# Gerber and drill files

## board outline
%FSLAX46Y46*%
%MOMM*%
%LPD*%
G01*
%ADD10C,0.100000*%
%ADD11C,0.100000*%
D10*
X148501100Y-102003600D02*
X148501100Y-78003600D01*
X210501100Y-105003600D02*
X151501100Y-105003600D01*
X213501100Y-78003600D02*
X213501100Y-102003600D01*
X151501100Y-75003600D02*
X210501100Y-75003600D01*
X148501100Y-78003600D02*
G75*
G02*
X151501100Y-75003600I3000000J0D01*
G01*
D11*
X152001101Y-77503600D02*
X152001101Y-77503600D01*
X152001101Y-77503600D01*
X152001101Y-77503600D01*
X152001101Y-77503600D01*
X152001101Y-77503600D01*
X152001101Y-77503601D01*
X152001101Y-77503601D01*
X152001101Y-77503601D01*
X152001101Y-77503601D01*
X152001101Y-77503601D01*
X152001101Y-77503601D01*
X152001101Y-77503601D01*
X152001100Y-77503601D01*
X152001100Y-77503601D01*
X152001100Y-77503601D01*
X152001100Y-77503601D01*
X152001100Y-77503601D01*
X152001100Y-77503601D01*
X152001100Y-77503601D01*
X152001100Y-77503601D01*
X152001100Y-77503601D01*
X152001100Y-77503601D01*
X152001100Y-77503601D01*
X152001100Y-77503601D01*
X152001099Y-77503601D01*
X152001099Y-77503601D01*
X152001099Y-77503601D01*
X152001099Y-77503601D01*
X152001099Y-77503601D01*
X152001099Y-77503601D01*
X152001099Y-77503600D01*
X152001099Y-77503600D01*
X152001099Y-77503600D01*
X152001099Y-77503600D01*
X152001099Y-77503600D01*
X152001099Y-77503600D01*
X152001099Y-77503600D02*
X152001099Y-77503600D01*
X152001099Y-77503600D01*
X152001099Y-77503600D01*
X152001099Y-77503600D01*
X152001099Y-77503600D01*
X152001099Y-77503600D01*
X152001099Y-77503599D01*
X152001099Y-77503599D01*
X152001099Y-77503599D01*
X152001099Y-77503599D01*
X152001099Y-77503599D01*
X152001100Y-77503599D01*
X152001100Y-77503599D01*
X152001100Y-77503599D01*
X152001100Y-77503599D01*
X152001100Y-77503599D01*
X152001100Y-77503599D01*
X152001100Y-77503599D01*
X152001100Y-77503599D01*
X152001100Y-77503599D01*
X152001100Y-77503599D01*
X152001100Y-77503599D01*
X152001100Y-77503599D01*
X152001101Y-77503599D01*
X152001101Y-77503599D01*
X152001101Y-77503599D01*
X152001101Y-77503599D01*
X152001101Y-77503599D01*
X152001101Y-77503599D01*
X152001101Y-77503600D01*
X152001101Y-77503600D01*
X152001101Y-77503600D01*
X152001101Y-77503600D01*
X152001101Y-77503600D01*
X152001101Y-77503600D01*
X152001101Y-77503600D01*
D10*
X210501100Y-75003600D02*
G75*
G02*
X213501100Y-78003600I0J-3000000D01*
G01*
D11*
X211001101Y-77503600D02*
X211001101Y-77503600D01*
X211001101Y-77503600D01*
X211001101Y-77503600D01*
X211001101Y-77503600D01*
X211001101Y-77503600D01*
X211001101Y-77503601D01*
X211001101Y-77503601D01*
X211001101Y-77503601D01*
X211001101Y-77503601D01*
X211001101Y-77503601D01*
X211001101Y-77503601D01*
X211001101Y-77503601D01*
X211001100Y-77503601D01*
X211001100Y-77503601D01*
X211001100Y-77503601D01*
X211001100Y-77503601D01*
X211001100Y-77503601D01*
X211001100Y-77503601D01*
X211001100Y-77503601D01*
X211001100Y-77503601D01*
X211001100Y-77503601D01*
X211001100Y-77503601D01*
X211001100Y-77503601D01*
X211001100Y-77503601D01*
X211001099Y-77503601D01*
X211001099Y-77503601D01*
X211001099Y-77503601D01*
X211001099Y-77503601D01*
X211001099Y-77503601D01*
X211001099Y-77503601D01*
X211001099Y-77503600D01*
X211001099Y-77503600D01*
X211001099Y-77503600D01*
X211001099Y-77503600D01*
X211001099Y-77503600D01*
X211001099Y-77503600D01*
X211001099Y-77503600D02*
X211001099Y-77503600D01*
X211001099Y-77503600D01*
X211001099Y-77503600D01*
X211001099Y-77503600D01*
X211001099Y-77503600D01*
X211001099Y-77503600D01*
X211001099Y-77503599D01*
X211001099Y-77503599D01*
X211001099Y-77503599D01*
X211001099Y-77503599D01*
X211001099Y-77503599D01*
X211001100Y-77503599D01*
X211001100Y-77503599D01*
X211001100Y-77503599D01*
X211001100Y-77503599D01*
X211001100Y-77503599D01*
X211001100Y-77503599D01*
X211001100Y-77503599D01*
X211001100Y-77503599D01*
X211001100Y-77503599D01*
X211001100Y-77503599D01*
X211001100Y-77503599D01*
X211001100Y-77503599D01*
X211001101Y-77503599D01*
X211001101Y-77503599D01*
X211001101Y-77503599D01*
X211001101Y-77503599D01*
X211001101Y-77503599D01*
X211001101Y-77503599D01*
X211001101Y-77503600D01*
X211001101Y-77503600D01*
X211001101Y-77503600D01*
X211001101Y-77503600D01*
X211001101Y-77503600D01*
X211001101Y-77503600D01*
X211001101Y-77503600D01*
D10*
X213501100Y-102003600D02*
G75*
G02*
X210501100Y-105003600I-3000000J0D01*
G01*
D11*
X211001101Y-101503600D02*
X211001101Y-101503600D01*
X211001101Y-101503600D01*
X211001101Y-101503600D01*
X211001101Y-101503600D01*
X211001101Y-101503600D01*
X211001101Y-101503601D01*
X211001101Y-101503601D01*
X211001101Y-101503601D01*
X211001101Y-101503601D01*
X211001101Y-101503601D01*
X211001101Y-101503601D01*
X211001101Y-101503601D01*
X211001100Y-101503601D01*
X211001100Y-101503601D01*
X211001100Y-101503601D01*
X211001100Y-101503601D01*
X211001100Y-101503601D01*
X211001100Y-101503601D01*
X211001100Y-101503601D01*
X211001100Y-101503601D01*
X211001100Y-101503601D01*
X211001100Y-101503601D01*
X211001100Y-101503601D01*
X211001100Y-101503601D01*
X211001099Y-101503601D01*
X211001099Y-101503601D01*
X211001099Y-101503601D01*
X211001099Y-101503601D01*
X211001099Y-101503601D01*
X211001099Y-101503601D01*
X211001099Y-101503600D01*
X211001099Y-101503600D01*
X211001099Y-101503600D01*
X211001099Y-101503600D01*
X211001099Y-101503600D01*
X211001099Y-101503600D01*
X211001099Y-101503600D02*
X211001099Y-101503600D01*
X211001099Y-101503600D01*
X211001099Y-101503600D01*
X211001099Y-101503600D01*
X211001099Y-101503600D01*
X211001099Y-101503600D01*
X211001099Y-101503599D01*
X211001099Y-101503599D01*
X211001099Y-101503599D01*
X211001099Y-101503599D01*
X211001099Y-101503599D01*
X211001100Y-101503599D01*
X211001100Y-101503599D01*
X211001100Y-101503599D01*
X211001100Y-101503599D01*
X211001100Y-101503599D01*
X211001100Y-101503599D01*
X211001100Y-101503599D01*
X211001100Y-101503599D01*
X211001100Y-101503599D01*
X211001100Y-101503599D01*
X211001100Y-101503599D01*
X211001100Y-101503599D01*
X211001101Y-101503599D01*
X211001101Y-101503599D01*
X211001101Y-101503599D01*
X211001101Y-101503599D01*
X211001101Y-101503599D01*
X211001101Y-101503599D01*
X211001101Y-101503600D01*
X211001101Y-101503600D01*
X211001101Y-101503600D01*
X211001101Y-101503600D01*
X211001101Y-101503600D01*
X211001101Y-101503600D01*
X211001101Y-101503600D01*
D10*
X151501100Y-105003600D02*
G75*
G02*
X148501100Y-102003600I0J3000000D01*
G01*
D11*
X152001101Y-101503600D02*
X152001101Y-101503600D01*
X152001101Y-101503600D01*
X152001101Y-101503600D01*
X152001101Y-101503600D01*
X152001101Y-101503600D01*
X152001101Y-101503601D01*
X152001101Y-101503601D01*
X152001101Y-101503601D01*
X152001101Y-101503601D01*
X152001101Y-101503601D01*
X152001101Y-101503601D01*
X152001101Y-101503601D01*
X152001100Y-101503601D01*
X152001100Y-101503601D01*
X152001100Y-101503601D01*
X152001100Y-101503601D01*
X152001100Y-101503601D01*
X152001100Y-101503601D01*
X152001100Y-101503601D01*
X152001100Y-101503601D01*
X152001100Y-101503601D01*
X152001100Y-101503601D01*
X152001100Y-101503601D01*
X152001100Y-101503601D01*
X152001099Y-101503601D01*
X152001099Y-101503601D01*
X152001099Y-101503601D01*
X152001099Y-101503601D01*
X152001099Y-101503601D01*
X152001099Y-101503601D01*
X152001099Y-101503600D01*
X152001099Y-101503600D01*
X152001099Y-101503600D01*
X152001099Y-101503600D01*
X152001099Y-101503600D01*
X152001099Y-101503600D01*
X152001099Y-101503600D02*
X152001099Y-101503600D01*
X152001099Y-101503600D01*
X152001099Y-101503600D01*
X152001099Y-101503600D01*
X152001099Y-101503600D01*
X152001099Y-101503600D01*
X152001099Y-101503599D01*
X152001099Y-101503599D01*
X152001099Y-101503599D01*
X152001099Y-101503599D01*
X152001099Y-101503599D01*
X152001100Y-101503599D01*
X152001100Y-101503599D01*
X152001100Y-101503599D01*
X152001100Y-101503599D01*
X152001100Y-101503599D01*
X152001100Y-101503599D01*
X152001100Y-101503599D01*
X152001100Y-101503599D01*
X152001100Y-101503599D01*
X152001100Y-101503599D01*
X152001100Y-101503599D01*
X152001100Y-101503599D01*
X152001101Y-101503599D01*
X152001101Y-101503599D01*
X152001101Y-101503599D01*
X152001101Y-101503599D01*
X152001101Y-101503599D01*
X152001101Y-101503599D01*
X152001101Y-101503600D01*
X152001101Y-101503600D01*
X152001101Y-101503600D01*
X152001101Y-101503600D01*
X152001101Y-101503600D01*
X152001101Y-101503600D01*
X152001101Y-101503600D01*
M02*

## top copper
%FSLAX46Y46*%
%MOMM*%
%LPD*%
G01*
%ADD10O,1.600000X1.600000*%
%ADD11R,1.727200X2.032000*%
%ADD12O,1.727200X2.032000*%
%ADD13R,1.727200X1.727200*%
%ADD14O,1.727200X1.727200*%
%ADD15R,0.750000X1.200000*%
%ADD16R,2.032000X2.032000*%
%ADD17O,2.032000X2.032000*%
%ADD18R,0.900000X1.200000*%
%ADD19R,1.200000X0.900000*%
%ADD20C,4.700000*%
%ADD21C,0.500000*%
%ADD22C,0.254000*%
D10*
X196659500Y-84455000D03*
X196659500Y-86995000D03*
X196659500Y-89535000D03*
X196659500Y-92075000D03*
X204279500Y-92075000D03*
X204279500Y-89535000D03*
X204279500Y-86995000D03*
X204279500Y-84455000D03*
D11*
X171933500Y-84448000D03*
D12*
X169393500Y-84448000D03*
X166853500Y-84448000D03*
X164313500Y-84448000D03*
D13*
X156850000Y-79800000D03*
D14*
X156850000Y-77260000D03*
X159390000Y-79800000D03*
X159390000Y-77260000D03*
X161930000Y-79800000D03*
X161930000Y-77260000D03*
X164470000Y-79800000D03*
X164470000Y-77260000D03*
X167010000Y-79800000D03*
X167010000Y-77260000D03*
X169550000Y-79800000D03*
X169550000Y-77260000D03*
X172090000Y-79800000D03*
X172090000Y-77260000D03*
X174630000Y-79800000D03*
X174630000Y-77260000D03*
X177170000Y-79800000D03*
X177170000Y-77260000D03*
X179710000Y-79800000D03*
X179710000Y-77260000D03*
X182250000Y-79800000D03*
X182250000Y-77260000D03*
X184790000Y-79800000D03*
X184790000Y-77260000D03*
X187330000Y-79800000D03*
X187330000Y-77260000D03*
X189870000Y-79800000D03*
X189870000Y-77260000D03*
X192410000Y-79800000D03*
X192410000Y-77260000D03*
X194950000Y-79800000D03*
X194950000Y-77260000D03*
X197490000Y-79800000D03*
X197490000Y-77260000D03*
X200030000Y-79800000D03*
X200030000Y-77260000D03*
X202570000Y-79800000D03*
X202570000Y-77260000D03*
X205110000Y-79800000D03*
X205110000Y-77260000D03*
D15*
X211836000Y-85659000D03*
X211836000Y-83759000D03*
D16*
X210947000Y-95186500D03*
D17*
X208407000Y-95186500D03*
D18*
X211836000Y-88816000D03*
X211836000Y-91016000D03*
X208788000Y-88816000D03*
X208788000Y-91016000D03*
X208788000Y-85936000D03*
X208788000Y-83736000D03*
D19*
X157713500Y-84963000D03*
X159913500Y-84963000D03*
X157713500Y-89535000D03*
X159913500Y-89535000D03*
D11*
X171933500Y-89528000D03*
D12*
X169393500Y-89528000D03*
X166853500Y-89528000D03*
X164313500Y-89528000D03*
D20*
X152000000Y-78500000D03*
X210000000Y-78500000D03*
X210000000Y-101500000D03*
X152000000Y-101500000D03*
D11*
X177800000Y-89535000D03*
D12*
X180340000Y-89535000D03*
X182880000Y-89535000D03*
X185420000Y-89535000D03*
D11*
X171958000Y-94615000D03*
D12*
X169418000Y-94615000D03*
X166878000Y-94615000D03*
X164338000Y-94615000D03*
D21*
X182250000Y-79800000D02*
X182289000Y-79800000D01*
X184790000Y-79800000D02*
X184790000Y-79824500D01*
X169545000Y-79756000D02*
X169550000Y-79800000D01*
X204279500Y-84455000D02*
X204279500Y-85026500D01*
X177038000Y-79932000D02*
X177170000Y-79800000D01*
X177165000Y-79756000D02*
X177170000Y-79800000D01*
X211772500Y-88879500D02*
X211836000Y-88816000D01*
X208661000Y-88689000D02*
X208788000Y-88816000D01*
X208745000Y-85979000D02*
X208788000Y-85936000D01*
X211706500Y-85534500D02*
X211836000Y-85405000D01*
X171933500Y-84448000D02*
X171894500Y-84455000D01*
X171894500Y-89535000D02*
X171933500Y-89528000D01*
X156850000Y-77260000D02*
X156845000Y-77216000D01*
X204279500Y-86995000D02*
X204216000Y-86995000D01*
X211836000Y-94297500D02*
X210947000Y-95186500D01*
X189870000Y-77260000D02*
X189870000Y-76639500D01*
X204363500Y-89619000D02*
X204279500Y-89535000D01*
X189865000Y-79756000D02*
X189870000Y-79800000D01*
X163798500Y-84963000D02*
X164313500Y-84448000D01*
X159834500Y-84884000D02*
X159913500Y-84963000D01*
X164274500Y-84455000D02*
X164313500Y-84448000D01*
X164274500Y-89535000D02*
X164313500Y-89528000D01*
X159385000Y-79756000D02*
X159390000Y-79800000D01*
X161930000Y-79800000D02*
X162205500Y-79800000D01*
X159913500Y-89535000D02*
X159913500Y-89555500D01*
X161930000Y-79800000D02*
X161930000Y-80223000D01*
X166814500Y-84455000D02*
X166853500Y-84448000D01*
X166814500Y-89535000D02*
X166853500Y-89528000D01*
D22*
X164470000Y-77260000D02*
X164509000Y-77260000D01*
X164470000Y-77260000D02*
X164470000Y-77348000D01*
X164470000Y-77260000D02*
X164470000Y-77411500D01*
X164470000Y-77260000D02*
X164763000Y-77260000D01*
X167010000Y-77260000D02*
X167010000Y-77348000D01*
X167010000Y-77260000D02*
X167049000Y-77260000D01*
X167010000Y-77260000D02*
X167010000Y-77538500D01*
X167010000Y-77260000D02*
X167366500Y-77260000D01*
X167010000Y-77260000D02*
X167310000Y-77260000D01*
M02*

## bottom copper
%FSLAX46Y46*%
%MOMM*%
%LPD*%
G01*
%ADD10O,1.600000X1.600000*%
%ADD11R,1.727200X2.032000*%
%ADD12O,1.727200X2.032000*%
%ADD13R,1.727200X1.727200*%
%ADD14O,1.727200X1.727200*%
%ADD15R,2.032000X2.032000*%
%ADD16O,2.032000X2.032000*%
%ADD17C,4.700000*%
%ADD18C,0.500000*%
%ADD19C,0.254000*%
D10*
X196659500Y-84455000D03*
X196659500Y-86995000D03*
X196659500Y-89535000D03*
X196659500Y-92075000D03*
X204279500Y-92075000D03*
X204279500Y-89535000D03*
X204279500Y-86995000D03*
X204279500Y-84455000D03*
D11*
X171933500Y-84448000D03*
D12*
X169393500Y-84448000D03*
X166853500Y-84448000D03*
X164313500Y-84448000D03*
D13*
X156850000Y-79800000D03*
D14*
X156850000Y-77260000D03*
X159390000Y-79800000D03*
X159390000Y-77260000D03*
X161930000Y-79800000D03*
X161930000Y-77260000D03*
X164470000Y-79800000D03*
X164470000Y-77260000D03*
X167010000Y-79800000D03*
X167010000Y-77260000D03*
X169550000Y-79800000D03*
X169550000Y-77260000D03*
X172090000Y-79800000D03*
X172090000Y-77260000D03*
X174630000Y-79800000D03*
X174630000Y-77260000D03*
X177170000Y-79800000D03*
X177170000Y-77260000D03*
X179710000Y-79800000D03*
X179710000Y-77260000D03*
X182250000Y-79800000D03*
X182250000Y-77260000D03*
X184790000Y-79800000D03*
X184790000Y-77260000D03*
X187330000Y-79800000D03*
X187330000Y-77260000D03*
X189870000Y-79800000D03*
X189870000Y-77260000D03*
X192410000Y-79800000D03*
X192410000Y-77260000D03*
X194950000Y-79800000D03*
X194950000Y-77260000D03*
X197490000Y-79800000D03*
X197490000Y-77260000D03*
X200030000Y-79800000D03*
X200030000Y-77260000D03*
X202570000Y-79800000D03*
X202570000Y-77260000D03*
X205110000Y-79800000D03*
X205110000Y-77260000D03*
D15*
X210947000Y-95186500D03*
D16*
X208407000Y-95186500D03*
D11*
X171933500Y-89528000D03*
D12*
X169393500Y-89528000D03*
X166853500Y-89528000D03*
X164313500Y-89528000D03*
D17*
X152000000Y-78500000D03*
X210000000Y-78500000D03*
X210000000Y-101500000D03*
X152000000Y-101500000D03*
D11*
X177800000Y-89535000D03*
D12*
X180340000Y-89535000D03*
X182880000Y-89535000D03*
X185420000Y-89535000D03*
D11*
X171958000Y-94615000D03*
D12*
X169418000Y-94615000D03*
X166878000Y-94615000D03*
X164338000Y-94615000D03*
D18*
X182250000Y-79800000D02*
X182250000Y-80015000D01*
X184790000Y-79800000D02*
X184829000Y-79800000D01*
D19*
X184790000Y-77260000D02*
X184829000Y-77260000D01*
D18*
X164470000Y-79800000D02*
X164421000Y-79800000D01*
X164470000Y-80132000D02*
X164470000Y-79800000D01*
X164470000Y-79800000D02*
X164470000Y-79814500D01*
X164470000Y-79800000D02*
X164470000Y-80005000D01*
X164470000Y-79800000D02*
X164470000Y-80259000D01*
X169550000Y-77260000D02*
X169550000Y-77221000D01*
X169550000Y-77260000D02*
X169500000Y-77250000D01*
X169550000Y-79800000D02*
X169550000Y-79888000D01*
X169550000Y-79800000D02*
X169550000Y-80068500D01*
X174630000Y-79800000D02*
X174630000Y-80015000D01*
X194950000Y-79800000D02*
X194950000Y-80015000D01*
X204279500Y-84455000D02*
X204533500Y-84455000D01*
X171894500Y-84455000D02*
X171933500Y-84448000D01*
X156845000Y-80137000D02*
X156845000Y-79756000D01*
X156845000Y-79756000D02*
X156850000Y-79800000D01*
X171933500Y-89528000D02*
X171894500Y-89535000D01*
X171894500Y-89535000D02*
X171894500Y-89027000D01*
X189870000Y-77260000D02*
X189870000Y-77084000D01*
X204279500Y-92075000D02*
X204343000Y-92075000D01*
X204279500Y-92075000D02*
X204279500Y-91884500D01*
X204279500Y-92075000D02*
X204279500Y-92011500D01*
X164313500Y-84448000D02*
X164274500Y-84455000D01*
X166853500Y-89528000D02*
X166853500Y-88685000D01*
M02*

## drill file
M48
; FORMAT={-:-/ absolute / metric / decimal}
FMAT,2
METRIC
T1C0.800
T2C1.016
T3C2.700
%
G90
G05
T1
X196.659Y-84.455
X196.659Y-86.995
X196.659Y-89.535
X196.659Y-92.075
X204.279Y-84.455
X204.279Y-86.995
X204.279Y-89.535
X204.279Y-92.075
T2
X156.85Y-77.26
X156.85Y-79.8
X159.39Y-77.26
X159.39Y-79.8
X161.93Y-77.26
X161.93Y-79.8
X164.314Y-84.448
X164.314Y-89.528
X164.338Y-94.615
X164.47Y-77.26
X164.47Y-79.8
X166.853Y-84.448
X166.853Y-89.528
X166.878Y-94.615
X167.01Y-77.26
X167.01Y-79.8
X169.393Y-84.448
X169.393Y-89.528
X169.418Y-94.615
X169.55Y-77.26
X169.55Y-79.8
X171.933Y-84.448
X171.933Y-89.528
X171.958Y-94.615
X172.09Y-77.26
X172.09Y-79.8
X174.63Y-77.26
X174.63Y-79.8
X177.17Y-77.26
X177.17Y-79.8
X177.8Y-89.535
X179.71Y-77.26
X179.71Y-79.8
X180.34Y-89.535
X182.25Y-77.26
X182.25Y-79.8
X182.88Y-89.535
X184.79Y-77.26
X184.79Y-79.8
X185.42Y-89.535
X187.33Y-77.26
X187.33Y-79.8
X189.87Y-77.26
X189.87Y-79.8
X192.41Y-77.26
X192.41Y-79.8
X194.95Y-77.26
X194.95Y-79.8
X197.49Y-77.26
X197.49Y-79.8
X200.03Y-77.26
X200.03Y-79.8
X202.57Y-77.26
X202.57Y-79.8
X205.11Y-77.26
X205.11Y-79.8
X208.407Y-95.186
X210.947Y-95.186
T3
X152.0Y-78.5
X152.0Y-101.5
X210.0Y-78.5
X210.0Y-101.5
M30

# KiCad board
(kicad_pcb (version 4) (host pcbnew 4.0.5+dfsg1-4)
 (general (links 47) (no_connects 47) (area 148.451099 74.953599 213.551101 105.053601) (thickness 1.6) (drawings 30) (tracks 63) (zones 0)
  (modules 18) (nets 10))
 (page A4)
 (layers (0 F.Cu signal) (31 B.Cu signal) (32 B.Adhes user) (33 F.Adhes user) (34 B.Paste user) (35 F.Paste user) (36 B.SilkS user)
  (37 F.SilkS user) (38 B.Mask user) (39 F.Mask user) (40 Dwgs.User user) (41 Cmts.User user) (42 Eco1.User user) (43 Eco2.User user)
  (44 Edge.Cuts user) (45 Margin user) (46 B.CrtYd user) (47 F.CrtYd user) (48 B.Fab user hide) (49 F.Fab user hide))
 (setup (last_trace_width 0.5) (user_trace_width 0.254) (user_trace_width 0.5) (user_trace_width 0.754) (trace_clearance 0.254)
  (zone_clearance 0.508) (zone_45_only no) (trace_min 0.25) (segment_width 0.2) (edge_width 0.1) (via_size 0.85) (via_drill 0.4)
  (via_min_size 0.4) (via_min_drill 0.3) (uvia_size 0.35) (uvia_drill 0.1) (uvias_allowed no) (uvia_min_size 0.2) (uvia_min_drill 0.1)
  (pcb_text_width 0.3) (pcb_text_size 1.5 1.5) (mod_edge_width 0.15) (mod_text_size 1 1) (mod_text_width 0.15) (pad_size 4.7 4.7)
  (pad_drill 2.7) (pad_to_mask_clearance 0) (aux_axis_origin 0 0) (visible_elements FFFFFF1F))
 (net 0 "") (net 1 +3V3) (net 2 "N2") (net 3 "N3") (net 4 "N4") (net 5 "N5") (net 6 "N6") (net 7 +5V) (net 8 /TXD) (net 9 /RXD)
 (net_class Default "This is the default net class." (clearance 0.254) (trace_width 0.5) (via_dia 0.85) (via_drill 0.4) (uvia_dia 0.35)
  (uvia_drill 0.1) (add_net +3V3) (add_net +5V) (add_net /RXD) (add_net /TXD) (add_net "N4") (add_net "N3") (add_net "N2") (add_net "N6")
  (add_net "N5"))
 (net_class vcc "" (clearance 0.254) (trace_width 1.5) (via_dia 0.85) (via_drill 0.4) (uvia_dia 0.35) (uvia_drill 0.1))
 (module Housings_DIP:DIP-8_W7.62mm (layer F.Cu) (at 196.6595 84.455)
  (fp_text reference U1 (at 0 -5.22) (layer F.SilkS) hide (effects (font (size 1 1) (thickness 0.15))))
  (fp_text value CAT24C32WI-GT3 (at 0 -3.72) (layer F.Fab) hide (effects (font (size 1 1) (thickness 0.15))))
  (pad 1 thru_hole oval (at 0 0) (size 1.6 1.6) (drill 0.8) (layers *.Cu *.Mask F.SilkS) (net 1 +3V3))
  (pad 2 thru_hole oval (at 0 2.54) (size 1.6 1.6) (drill 0.8) (layers *.Cu *.Mask F.SilkS) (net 1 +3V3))
  (pad 3 thru_hole oval (at 0 5.08) (size 1.6 1.6) (drill 0.8) (layers *.Cu *.Mask F.SilkS) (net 1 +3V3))
  (pad 4 thru_hole oval (at 0 7.62) (size 1.6 1.6) (drill 0.8) (layers *.Cu *.Mask F.SilkS) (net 1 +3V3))
  (pad 5 thru_hole oval (at 7.62 7.62) (size 1.6 1.6) (drill 0.8) (layers *.Cu *.Mask F.SilkS) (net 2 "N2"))
  (pad 6 thru_hole oval (at 7.62 5.08) (size 1.6 1.6) (drill 0.8) (layers *.Cu *.Mask F.SilkS) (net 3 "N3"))
  (pad 7 thru_hole oval (at 7.62 2.54) (size 1.6 1.6) (drill 0.8) (layers *.Cu *.Mask F.SilkS) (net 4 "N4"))
  (pad 8 thru_hole oval (at 7.62 0) (size 1.6 1.6) (drill 0.8) (layers *.Cu *.Mask F.SilkS) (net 1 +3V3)))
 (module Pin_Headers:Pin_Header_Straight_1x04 (layer F.Cu) (at 171.9335 84.448 270)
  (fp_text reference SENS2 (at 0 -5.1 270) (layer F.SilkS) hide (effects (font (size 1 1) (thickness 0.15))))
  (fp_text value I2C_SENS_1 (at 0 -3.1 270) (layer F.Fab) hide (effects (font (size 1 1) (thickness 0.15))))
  (pad 1 thru_hole rect (at 0 0 270) (size 2.032 1.7272) (drill 1.016) (layers *.Cu *.Mask F.SilkS) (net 1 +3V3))
  (pad 2 thru_hole oval (at 0 2.54 270) (size 2.032 1.7272) (drill 1.016) (layers *.Cu *.Mask F.SilkS) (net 1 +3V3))
  (pad 3 thru_hole oval (at 0 5.08 270) (size 2.032 1.7272) (drill 1.016) (layers *.Cu *.Mask F.SilkS) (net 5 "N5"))
  (pad 4 thru_hole oval (at 0 7.62 270) (size 2.032 1.7272) (drill 1.016) (layers *.Cu *.Mask F.SilkS) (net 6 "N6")))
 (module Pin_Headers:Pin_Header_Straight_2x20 (layer F.Cu) (at 156.85 79.8 90)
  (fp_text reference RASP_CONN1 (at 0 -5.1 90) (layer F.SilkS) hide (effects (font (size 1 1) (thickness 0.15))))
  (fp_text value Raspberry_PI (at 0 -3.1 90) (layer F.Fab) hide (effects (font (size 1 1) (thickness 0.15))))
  (pad 1 thru_hole rect (at 0 0 90) (size 1.7272 1.7272) (drill 1.016) (layers *.Cu *.Mask F.SilkS) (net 1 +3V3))
  (pad 2 thru_hole oval (at 2.54 0 90) (size 1.7272 1.7272) (drill 1.016) (layers *.Cu *.Mask F.SilkS) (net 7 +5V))
  (pad 3 thru_hole oval (at 0 2.54 90) (size 1.7272 1.7272) (drill 1.016) (layers *.Cu *.Mask F.SilkS) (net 6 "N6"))
  (pad 4 thru_hole oval (at 2.54 2.54 90) (size 1.7272 1.7272) (drill 1.016) (layers *.Cu *.Mask F.SilkS) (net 7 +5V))
  (pad 5 thru_hole oval (at 0 5.08 90) (size 1.7272 1.7272) (drill 1.016) (layers *.Cu *.Mask F.SilkS) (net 5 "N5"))
  (pad 6 thru_hole oval (at 2.54 5.08 90) (size 1.7272 1.7272) (drill 1.016) (layers *.Cu *.Mask F.SilkS) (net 1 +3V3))
  (pad 7 thru_hole oval (at 0 7.62 90) (size 1.7272 1.7272) (drill 1.016) (layers *.Cu *.Mask F.SilkS))
  (pad 8 thru_hole oval (at 2.54 7.62 90) (size 1.7272 1.7272) (drill 1.016) (layers *.Cu *.Mask F.SilkS) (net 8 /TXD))
  (pad 9 thru_hole oval (at 0 10.16 90) (size 1.7272 1.7272) (drill 1.016) (layers *.Cu *.Mask F.SilkS) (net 1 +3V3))
  (pad 10 thru_hole oval (at 2.54 10.16 90) (size 1.7272 1.7272) (drill 1.016) (layers *.Cu *.Mask F.SilkS) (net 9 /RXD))
  (pad 11 thru_hole oval (at 0 12.7 90) (size 1.7272 1.7272) (drill 1.016) (layers *.Cu *.Mask F.SilkS))
  (pad 12 thru_hole oval (at 2.54 12.7 90) (size 1.7272 1.7272) (drill 1.016) (layers *.Cu *.Mask F.SilkS))
  (pad 13 thru_hole oval (at 0 15.24 90) (size 1.7272 1.7272) (drill 1.016) (layers *.Cu *.Mask F.SilkS))
  (pad 14 thru_hole oval (at 2.54 15.24 90) (size 1.7272 1.7272) (drill 1.016) (layers *.Cu *.Mask F.SilkS) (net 1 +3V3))
  (pad 15 thru_hole oval (at 0 17.78 90) (size 1.7272 1.7272) (drill 1.016) (layers *.Cu *.Mask F.SilkS))
  (pad 16 thru_hole oval (at 2.54 17.78 90) (size 1.7272 1.7272) (drill 1.016) (layers *.Cu *.Mask F.SilkS))
  (pad 17 thru_hole oval (at 0 20.32 90) (size 1.7272 1.7272) (drill 1.016) (layers *.Cu *.Mask F.SilkS) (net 1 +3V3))
  (pad 18 thru_hole oval (at 2.54 20.32 90) (size 1.7272 1.7272) (drill 1.016) (layers *.Cu *.Mask F.SilkS))
  (pad 19 thru_hole oval (at 0 22.86 90) (size 1.7272 1.7272) (drill 1.016) (layers *.Cu *.Mask F.SilkS))
  (pad 20 thru_hole oval (at 2.54 22.86 90) (size 1.7272 1.7272) (drill 1.016) (layers *.Cu *.Mask F.SilkS) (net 1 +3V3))
  (pad 21 thru_hole oval (at 0 25.4 90) (size 1.7272 1.7272) (drill 1.016) (layers *.Cu *.Mask F.SilkS))
  (pad 22 thru_hole oval (at 2.54 25.4 90) (size 1.7272 1.7272) (drill 1.016) (layers *.Cu *.Mask F.SilkS))
  (pad 23 thru_hole oval (at 0 27.94 90) (size 1.7272 1.7272) (drill 1.016) (layers *.Cu *.Mask F.SilkS))
  (pad 24 thru_hole oval (at 2.54 27.94 90) (size 1.7272 1.7272) (drill 1.016) (layers *.Cu *.Mask F.SilkS))
  (pad 25 thru_hole oval (at 0 30.48 90) (size 1.7272 1.7272) (drill 1.016) (layers *.Cu *.Mask F.SilkS) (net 1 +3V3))
  (pad 26 thru_hole oval (at 2.54 30.48 90) (size 1.7272 1.7272) (drill 1.016) (layers *.Cu *.Mask F.SilkS))
  (pad 27 thru_hole oval (at 0 33.02 90) (size 1.7272 1.7272) (drill 1.016) (layers *.Cu *.Mask F.SilkS) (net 2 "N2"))
  (pad 28 thru_hole oval (at 2.54 33.02 90) (size 1.7272 1.7272) (drill 1.016) (layers *.Cu *.Mask F.SilkS) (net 3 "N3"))
  (pad 29 thru_hole oval (at 0 35.56 90) (size 1.7272 1.7272) (drill 1.016) (layers *.Cu *.Mask F.SilkS))
  (pad 30 thru_hole oval (at 2.54 35.56 90) (size 1.7272 1.7272) (drill 1.016) (layers *.Cu *.Mask F.SilkS) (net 1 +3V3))
  (pad 31 thru_hole oval (at 0 38.1 90) (size 1.7272 1.7272) (drill 1.016) (layers *.Cu *.Mask F.SilkS))
  (pad 32 thru_hole oval (at 2.54 38.1 90) (size 1.7272 1.7272) (drill 1.016) (layers *.Cu *.Mask F.SilkS))
  (pad 33 thru_hole oval (at 0 40.64 90) (size 1.7272 1.7272) (drill 1.016) (layers *.Cu *.Mask F.SilkS))
  (pad 34 thru_hole oval (at 2.54 40.64 90) (size 1.7272 1.7272) (drill 1.016) (layers *.Cu *.Mask F.SilkS) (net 1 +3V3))
  (pad 35 thru_hole oval (at 0 43.18 90) (size 1.7272 1.7272) (drill 1.016) (layers *.Cu *.Mask F.SilkS))
  (pad 36 thru_hole oval (at 2.54 43.18 90) (size 1.7272 1.7272) (drill 1.016) (layers *.Cu *.Mask F.SilkS))
  (pad 37 thru_hole oval (at 0 45.72 90) (size 1.7272 1.7272) (drill 1.016) (layers *.Cu *.Mask F.SilkS))
  (pad 38 thru_hole oval (at 2.54 45.72 90) (size 1.7272 1.7272) (drill 1.016) (layers *.Cu *.Mask F.SilkS))
  (pad 39 thru_hole oval (at 0 48.26 90) (size 1.7272 1.7272) (drill 1.016) (layers *.Cu *.Mask F.SilkS) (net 1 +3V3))
  (pad 40 thru_hole oval (at 2.54 48.26 90) (size 1.7272 1.7272) (drill 1.016) (layers *.Cu *.Mask F.SilkS)))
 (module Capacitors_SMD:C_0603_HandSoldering (layer F.Cu) (at 211.836 84.709 90)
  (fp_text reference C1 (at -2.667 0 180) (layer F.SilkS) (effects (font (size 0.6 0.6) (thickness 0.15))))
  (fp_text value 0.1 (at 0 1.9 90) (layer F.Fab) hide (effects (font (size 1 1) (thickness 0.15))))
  (pad 1 smd rect (at -0.95 0 90) (size 1.2 0.75) (layers F.Cu F.Paste F.Mask) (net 1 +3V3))
  (pad 2 smd rect (at 0.95 0 90) (size 1.2 0.75) (layers F.Cu F.Paste F.Mask) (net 1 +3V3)))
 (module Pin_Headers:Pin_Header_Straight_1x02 (layer F.Cu) (at 210.947 95.1865 270)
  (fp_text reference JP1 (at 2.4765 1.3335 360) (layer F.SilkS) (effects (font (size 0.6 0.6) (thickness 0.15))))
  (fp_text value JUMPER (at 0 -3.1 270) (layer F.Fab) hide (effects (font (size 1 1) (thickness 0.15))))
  (pad 1 thru_hole rect (at 0 0 270) (size 2.032 2.032) (drill 1.016) (layers *.Cu *.Mask F.SilkS) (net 4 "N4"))
  (pad 2 thru_hole oval (at 0 2.54 270) (size 2.032 2.032) (drill 1.016) (layers *.Cu *.Mask F.SilkS) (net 1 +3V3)))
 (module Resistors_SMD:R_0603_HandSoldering (layer F.Cu) (at 211.836 89.916 270)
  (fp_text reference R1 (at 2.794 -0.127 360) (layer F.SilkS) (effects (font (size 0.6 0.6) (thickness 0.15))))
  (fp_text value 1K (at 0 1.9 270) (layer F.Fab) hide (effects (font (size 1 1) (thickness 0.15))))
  (pad 1 smd rect (at -1.1 0 270) (size 1.2 0.9) (layers F.Cu F.Paste F.Mask) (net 1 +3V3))
  (pad 2 smd rect (at 1.1 0 270) (size 1.2 0.9) (layers F.Cu F.Paste F.Mask) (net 4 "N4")))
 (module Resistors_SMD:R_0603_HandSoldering (layer F.Cu) (at 208.788 89.916 270)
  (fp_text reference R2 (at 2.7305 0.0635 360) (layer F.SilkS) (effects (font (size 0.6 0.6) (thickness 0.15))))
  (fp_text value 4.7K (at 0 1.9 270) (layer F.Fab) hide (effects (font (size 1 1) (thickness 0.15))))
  (pad 1 smd rect (at -1.1 0 270) (size 1.2 0.9) (layers F.Cu F.Paste F.Mask) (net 1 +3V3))
  (pad 2 smd rect (at 1.1 0 270) (size 1.2 0.9) (layers F.Cu F.Paste F.Mask) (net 3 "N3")))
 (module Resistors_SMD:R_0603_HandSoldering (layer F.Cu) (at 208.788 84.836 90)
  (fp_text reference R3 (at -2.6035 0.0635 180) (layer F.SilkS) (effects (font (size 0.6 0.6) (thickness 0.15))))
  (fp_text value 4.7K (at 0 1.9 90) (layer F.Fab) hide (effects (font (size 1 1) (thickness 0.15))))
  (pad 1 smd rect (at -1.1 0 90) (size 1.2 0.9) (layers F.Cu F.Paste F.Mask) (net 1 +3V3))
  (pad 2 smd rect (at 1.1 0 90) (size 1.2 0.9) (layers F.Cu F.Paste F.Mask) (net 2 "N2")))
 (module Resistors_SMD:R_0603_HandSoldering (layer F.Cu) (at 158.8135 84.963)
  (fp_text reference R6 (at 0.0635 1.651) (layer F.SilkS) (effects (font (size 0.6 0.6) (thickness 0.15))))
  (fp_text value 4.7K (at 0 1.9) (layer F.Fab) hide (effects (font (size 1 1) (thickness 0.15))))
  (pad 1 smd rect (at -1.1 0) (size 1.2 0.9) (layers F.Cu F.Paste F.Mask) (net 1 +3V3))
  (pad 2 smd rect (at 1.1 0) (size 1.2 0.9) (layers F.Cu F.Paste F.Mask) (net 6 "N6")))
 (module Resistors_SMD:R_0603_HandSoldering (layer F.Cu) (at 158.8135 89.535)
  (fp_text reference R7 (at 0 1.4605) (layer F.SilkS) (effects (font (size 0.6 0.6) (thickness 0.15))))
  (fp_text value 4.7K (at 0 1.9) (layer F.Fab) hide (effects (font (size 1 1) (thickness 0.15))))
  (pad 1 smd rect (at -1.1 0) (size 1.2 0.9) (layers F.Cu F.Paste F.Mask) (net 1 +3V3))
  (pad 2 smd rect (at 1.1 0) (size 1.2 0.9) (layers F.Cu F.Paste F.Mask) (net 5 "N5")))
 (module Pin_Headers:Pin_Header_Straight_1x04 (layer F.Cu) (at 171.9335 89.528 270)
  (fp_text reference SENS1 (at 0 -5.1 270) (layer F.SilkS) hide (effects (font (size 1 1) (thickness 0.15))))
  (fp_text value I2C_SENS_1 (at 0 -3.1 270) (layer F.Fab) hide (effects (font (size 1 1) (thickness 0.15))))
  (pad 1 thru_hole rect (at 0 0 270) (size 2.032 1.7272) (drill 1.016) (layers *.Cu *.Mask F.SilkS) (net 1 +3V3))
  (pad 2 thru_hole oval (at 0 2.54 270) (size 2.032 1.7272) (drill 1.016) (layers *.Cu *.Mask F.SilkS) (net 1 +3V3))
  (pad 3 thru_hole oval (at 0 5.08 270) (size 2.032 1.7272) (drill 1.016) (layers *.Cu *.Mask F.SilkS) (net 5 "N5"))
  (pad 4 thru_hole oval (at 0 7.62 270) (size 2.032 1.7272) (drill 1.016) (layers *.Cu *.Mask F.SilkS) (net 6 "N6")))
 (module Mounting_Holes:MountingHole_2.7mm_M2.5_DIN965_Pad (layer F.Cu) (at 152 78.5)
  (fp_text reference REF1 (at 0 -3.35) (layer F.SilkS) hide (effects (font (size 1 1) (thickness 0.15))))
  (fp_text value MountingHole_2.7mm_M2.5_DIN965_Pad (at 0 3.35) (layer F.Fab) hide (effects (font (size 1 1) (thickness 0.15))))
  (pad 1 thru_hole circle (at 0 0) (size 4.7 4.7) (drill 2.7) (layers *.Cu *.Mask F.SilkS)))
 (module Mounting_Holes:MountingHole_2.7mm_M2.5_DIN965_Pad (layer F.Cu) (at 210 78.5)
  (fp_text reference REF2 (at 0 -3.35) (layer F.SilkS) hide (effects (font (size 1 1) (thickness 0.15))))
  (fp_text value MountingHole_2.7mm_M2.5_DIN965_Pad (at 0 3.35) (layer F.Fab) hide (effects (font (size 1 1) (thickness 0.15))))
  (pad 2 thru_hole circle (at 0 0) (size 4.7 4.7) (drill 2.7) (layers *.Cu *.Mask F.SilkS)))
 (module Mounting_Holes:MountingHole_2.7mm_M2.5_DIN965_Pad (layer F.Cu) (at 210 101.5)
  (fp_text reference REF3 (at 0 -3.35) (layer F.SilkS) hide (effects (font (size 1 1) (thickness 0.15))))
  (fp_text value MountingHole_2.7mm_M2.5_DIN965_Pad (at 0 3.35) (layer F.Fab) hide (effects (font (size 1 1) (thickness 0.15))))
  (pad 3 thru_hole circle (at 0 0) (size 4.7 4.7) (drill 2.7) (layers *.Cu *.Mask F.SilkS)))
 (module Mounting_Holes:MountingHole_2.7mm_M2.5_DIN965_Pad (layer F.Cu) (at 152 101.5)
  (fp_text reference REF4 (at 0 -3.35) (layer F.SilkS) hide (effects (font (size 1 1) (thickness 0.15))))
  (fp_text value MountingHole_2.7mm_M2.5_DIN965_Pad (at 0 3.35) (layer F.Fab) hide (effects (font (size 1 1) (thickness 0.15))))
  (pad 4 thru_hole circle (at 0 0) (size 4.7 4.7) (drill 2.7) (layers *.Cu *.Mask F.SilkS)))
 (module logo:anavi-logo (layer F.Cu) (at 176.7205 84.201)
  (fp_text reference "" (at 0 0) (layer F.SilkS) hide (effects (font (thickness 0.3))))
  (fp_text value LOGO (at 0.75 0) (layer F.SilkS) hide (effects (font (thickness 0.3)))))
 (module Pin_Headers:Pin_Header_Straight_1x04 (layer F.Cu) (at 177.8 89.535 90)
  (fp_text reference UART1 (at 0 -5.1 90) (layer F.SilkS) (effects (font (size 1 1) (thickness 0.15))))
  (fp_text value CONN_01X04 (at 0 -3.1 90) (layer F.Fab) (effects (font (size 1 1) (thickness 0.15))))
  (pad 1 thru_hole rect (at 0 0 90) (size 2.032 1.7272) (drill 1.016) (layers *.Cu *.Mask) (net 1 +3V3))
  (pad 2 thru_hole oval (at 0 2.54 90) (size 2.032 1.7272) (drill 1.016) (layers *.Cu *.Mask) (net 8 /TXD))
  (pad 3 thru_hole oval (at 0 5.08 90) (size 2.032 1.7272) (drill 1.016) (layers *.Cu *.Mask) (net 9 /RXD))
  (pad 4 thru_hole oval (at 0 7.62 90) (size 2.032 1.7272) (drill 1.016) (layers *.Cu *.Mask) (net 1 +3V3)))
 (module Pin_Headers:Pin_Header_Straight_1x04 (layer F.Cu) (at 171.958 94.615 270)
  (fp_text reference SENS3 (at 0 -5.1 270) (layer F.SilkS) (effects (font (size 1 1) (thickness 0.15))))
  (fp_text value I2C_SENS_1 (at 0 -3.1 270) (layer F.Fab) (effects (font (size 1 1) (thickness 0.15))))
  (pad 1 thru_hole rect (at 0 0 270) (size 2.032 1.7272) (drill 1.016) (layers *.Cu *.Mask) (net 1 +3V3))
  (pad 2 thru_hole oval (at 0 2.54 270) (size 2.032 1.7272) (drill 1.016) (layers *.Cu *.Mask) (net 1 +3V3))
  (pad 3 thru_hole oval (at 0 5.08 270) (size 2.032 1.7272) (drill 1.016) (layers *.Cu *.Mask) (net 5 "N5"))
  (pad 4 thru_hole oval (at 0 7.62 270) (size 2.032 1.7272) (drill 1.016) (layers *.Cu *.Mask) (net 6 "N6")))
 (gr_line (start 148.5011 102.0036) (end 148.5011 78.0036) (layer Edge.Cuts) (width 0.1))
 (gr_line (start 210.5011 105.0036) (end 151.5011 105.0036) (layer Edge.Cuts) (width 0.1))
 (gr_line (start 213.5011 78.0036) (end 213.5011 102.0036) (layer Edge.Cuts) (width 0.1))
 (gr_line (start 151.5011 75.0036) (end 210.5011 75.0036) (layer Edge.Cuts) (width 0.1))
 (gr_arc (start 151.5011 78.0036) (end 151.5011 75.0036) (angle -90) (layer Edge.Cuts) (width 0.1))
 (gr_circle (center 152.0011 77.5036) (end 152.0011 77.5036) (layer Edge.Cuts) (width 0.1))
 (gr_arc (start 210.5011 78.0036) (end 213.5011 78.0036) (angle -90) (layer Edge.Cuts) (width 0.1))
 (gr_circle (center 211.0011 77.5036) (end 211.0011 77.5036) (layer Edge.Cuts) (width 0.1))
 (gr_arc (start 210.5011 102.0036) (end 210.5011 105.0036) (angle -90) (layer Edge.Cuts) (width 0.1))
 (gr_circle (center 211.0011 101.5036) (end 211.0011 101.5036) (layer Edge.Cuts) (width 0.1))
 (gr_arc (start 151.5011 102.0036) (end 148.5011 102.0036) (angle -90) (layer Edge.Cuts) (width 0.1))
 (gr_circle (center 152.0011 101.5036) (end 152.0011 101.5036) (layer Edge.Cuts) (width 0.1))
 (segment (start 182.25 79.8) (end 182.289 79.8) (width 0.5) (layer F.Cu) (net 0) (status 30))
 (segment (start 182.25 79.8) (end 182.25 80.015) (width 0.5) (layer B.Cu) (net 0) (status 30))
 (segment (start 184.79 79.8) (end 184.829 79.8) (width 0.5) (layer B.Cu) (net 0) (status 30))
 (segment (start 184.79 79.8) (end 184.79 79.8245) (width 0.5) (layer F.Cu) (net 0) (status 30))
 (segment (start 184.79 77.26) (end 184.829 77.26) (width 0.254) (layer B.Cu) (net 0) (status 30))
 (segment (start 164.47 79.8) (end 164.421 79.8) (width 0.5) (layer B.Cu) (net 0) (status 30))
 (segment (start 164.47 80.132) (end 164.47 79.8) (width 0.5) (layer B.Cu) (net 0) (status 30))
 (segment (start 164.47 79.8) (end 164.47 79.8145) (width 0.5) (layer B.Cu) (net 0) (status 30))
 (segment (start 164.47 79.8) (end 164.47 80.005) (width 0.5) (layer B.Cu) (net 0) (status 30))
 (segment (start 164.47 79.8) (end 164.47 80.259) (width 0.5) (layer B.Cu) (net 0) (status 30))
 (segment (start 169.55 77.26) (end 169.55 77.221) (width 0.5) (layer B.Cu) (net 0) (status 30))
 (segment (start 169.55 77.26) (end 169.5 77.25) (width 0.5) (layer B.Cu) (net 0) (status 80030))
 (segment (start 169.55 79.8) (end 169.55 79.888) (width 0.5) (layer B.Cu) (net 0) (status 30))
 (segment (start 169.545 79.756) (end 169.55 79.8) (width 0.5) (layer F.Cu) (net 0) (status 80030))
 (segment (start 169.55 79.8) (end 169.55 80.0685) (width 0.5) (layer B.Cu) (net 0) (status 30))
 (segment (start 174.63 79.8) (end 174.63 80.015) (width 0.5) (layer B.Cu) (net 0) (status 30))
 (segment (start 194.95 79.8) (end 194.95 80.015) (width 0.5) (layer B.Cu) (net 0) (status 30))
 (segment (start 204.2795 84.455) (end 204.5335 84.455) (width 0.5) (layer B.Cu) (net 1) (status 30))
 (segment (start 204.2795 84.455) (end 204.2795 85.0265) (width 0.5) (layer F.Cu) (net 1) (status 30))
 (segment (start 177.038 79.932) (end 177.17 79.8) (width 0.5) (layer F.Cu) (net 1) (status 30))
 (segment (start 177.165 79.756) (end 177.17 79.8) (width 0.5) (layer F.Cu) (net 1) (status 80030))
 (segment (start 171.8945 84.455) (end 171.9335 84.448) (width 0.5) (layer B.Cu) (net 1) (status 80030))
 (segment (start 211.7725 88.8795) (end 211.836 88.816) (width 0.5) (layer F.Cu) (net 1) (status 30))
 (segment (start 208.661 88.689) (end 208.788 88.816) (width 0.5) (layer F.Cu) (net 1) (status 30))
 (segment (start 208.745 85.979) (end 208.788 85.936) (width 0.5) (layer F.Cu) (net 1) (status 30))
 (segment (start 211.7065 85.5345) (end 211.836 85.405) (width 0.5) (layer F.Cu) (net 1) (status 30))
 (segment (start 156.845 80.137) (end 156.845 79.756) (width 0.5) (layer B.Cu) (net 1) (status 80030))
 (segment (start 156.845 79.756) (end 156.85 79.8) (width 0.5) (layer B.Cu) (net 1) (status 80030))
 (segment (start 171.9335 89.528) (end 171.8945 89.535) (width 0.5) (layer B.Cu) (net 1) (status 80030))
 (segment (start 171.8945 89.535) (end 171.8945 89.027) (width 0.5) (layer B.Cu) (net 1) (status 80030))
 (segment (start 171.9335 84.448) (end 171.8945 84.455) (width 0.5) (layer F.Cu) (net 1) (status 80030))
 (segment (start 171.8945 89.535) (end 171.9335 89.528) (width 0.5) (layer F.Cu) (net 1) (status 80030))
 (segment (start 156.85 77.26) (end 156.845 77.216) (width 0.5) (layer F.Cu) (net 7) (status 80030))
 (segment (start 204.2795 86.995) (end 204.216 86.995) (width 0.5) (layer F.Cu) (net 4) (status 30))
 (segment (start 211.836 94.2975) (end 210.947 95.1865) (width 0.5) (layer F.Cu) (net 4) (status 30))
 (segment (start 189.87 77.26) (end 189.87 76.6395) (width 0.5) (layer F.Cu) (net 3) (status 30))
 (segment (start 189.87 77.26) (end 189.87 77.084) (width 0.5) (layer B.Cu) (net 3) (status 30))
 (segment (start 204.3635 89.619) (end 204.2795 89.535) (width 0.5) (layer F.Cu) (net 3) (status 30))
 (segment (start 204.2795 92.075) (end 204.343 92.075) (width 0.5) (layer B.Cu) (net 2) (status 30))
 (segment (start 204.2795 92.075) (end 204.2795 91.8845) (width 0.5) (layer B.Cu) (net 2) (status 30))
 (segment (start 204.2795 92.075) (end 204.2795 92.0115) (width 0.5) (layer B.Cu) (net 2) (status 30))
 (segment (start 189.865 79.756) (end 189.87 79.8) (width 0.5) (layer F.Cu) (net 2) (status 80030))
 (segment (start 164.3135 84.448) (end 164.2745 84.455) (width 0.5) (layer B.Cu) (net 6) (status 80030))
 (segment (start 163.7985 84.963) (end 164.3135 84.448) (width 0.5) (layer F.Cu) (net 6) (status 30))
 (segment (start 159.8345 84.884) (end 159.9135 84.963) (width 0.5) (layer F.Cu) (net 6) (status 30))
 (segment (start 164.2745 84.455) (end 164.3135 84.448) (width 0.5) (layer F.Cu) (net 6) (status 80030))
 (segment (start 164.2745 89.535) (end 164.3135 89.528) (width 0.5) (layer F.Cu) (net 6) (status 80030))
 (segment (start 159.385 79.756) (end 159.39 79.8) (width 0.5) (layer F.Cu) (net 6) (status 80030))
 (segment (start 161.93 79.8) (end 162.2055 79.8) (width 0.5) (layer F.Cu) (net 5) (status 30))
 (segment (start 159.9135 89.535) (end 159.9135 89.5555) (width 0.5) (layer F.Cu) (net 5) (status 30))
 (segment (start 161.93 79.8) (end 161.93 80.223) (width 0.5) (layer F.Cu) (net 5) (status 30))
 (segment (start 166.8535 89.528) (end 166.8535 88.685) (width 0.5) (layer B.Cu) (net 5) (status 30))
 (segment (start 166.8145 84.455) (end 166.8535 84.448) (width 0.5) (layer F.Cu) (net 5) (status 80030))
 (segment (start 166.8145 89.535) (end 166.8535 89.528) (width 0.5) (layer F.Cu) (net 5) (status 80030))
 (segment (start 164.47 77.26) (end 164.509 77.26) (width 0.254) (layer F.Cu) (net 8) (status 30))
 (segment (start 164.47 77.26) (end 164.47 77.348) (width 0.254) (layer F.Cu) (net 8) (status 30))
 (segment (start 164.47 77.26) (end 164.47 77.4115) (width 0.254) (layer F.Cu) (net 8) (status 30))
 (segment (start 164.47 77.26) (end 164.763 77.26) (width 0.254) (layer F.Cu) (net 8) (status 30))
 (segment (start 167.01 77.26) (end 167.01 77.348) (width 0.254) (layer F.Cu) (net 9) (status 30))
 (segment (start 167.01 77.26) (end 167.049 77.26) (width 0.254) (layer F.Cu) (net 9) (status 30))
 (segment (start 167.01 77.26) (end 167.01 77.5385) (width 0.254) (layer F.Cu) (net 9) (status 30))
 (segment (start 167.01 77.26) (end 167.3665 77.26) (width 0.254) (layer F.Cu) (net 9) (status 30))
 (segment (start 167.01 77.26) (end 167.31 77.26) (width 0.254) (layer F.Cu) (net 9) (status 30)))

